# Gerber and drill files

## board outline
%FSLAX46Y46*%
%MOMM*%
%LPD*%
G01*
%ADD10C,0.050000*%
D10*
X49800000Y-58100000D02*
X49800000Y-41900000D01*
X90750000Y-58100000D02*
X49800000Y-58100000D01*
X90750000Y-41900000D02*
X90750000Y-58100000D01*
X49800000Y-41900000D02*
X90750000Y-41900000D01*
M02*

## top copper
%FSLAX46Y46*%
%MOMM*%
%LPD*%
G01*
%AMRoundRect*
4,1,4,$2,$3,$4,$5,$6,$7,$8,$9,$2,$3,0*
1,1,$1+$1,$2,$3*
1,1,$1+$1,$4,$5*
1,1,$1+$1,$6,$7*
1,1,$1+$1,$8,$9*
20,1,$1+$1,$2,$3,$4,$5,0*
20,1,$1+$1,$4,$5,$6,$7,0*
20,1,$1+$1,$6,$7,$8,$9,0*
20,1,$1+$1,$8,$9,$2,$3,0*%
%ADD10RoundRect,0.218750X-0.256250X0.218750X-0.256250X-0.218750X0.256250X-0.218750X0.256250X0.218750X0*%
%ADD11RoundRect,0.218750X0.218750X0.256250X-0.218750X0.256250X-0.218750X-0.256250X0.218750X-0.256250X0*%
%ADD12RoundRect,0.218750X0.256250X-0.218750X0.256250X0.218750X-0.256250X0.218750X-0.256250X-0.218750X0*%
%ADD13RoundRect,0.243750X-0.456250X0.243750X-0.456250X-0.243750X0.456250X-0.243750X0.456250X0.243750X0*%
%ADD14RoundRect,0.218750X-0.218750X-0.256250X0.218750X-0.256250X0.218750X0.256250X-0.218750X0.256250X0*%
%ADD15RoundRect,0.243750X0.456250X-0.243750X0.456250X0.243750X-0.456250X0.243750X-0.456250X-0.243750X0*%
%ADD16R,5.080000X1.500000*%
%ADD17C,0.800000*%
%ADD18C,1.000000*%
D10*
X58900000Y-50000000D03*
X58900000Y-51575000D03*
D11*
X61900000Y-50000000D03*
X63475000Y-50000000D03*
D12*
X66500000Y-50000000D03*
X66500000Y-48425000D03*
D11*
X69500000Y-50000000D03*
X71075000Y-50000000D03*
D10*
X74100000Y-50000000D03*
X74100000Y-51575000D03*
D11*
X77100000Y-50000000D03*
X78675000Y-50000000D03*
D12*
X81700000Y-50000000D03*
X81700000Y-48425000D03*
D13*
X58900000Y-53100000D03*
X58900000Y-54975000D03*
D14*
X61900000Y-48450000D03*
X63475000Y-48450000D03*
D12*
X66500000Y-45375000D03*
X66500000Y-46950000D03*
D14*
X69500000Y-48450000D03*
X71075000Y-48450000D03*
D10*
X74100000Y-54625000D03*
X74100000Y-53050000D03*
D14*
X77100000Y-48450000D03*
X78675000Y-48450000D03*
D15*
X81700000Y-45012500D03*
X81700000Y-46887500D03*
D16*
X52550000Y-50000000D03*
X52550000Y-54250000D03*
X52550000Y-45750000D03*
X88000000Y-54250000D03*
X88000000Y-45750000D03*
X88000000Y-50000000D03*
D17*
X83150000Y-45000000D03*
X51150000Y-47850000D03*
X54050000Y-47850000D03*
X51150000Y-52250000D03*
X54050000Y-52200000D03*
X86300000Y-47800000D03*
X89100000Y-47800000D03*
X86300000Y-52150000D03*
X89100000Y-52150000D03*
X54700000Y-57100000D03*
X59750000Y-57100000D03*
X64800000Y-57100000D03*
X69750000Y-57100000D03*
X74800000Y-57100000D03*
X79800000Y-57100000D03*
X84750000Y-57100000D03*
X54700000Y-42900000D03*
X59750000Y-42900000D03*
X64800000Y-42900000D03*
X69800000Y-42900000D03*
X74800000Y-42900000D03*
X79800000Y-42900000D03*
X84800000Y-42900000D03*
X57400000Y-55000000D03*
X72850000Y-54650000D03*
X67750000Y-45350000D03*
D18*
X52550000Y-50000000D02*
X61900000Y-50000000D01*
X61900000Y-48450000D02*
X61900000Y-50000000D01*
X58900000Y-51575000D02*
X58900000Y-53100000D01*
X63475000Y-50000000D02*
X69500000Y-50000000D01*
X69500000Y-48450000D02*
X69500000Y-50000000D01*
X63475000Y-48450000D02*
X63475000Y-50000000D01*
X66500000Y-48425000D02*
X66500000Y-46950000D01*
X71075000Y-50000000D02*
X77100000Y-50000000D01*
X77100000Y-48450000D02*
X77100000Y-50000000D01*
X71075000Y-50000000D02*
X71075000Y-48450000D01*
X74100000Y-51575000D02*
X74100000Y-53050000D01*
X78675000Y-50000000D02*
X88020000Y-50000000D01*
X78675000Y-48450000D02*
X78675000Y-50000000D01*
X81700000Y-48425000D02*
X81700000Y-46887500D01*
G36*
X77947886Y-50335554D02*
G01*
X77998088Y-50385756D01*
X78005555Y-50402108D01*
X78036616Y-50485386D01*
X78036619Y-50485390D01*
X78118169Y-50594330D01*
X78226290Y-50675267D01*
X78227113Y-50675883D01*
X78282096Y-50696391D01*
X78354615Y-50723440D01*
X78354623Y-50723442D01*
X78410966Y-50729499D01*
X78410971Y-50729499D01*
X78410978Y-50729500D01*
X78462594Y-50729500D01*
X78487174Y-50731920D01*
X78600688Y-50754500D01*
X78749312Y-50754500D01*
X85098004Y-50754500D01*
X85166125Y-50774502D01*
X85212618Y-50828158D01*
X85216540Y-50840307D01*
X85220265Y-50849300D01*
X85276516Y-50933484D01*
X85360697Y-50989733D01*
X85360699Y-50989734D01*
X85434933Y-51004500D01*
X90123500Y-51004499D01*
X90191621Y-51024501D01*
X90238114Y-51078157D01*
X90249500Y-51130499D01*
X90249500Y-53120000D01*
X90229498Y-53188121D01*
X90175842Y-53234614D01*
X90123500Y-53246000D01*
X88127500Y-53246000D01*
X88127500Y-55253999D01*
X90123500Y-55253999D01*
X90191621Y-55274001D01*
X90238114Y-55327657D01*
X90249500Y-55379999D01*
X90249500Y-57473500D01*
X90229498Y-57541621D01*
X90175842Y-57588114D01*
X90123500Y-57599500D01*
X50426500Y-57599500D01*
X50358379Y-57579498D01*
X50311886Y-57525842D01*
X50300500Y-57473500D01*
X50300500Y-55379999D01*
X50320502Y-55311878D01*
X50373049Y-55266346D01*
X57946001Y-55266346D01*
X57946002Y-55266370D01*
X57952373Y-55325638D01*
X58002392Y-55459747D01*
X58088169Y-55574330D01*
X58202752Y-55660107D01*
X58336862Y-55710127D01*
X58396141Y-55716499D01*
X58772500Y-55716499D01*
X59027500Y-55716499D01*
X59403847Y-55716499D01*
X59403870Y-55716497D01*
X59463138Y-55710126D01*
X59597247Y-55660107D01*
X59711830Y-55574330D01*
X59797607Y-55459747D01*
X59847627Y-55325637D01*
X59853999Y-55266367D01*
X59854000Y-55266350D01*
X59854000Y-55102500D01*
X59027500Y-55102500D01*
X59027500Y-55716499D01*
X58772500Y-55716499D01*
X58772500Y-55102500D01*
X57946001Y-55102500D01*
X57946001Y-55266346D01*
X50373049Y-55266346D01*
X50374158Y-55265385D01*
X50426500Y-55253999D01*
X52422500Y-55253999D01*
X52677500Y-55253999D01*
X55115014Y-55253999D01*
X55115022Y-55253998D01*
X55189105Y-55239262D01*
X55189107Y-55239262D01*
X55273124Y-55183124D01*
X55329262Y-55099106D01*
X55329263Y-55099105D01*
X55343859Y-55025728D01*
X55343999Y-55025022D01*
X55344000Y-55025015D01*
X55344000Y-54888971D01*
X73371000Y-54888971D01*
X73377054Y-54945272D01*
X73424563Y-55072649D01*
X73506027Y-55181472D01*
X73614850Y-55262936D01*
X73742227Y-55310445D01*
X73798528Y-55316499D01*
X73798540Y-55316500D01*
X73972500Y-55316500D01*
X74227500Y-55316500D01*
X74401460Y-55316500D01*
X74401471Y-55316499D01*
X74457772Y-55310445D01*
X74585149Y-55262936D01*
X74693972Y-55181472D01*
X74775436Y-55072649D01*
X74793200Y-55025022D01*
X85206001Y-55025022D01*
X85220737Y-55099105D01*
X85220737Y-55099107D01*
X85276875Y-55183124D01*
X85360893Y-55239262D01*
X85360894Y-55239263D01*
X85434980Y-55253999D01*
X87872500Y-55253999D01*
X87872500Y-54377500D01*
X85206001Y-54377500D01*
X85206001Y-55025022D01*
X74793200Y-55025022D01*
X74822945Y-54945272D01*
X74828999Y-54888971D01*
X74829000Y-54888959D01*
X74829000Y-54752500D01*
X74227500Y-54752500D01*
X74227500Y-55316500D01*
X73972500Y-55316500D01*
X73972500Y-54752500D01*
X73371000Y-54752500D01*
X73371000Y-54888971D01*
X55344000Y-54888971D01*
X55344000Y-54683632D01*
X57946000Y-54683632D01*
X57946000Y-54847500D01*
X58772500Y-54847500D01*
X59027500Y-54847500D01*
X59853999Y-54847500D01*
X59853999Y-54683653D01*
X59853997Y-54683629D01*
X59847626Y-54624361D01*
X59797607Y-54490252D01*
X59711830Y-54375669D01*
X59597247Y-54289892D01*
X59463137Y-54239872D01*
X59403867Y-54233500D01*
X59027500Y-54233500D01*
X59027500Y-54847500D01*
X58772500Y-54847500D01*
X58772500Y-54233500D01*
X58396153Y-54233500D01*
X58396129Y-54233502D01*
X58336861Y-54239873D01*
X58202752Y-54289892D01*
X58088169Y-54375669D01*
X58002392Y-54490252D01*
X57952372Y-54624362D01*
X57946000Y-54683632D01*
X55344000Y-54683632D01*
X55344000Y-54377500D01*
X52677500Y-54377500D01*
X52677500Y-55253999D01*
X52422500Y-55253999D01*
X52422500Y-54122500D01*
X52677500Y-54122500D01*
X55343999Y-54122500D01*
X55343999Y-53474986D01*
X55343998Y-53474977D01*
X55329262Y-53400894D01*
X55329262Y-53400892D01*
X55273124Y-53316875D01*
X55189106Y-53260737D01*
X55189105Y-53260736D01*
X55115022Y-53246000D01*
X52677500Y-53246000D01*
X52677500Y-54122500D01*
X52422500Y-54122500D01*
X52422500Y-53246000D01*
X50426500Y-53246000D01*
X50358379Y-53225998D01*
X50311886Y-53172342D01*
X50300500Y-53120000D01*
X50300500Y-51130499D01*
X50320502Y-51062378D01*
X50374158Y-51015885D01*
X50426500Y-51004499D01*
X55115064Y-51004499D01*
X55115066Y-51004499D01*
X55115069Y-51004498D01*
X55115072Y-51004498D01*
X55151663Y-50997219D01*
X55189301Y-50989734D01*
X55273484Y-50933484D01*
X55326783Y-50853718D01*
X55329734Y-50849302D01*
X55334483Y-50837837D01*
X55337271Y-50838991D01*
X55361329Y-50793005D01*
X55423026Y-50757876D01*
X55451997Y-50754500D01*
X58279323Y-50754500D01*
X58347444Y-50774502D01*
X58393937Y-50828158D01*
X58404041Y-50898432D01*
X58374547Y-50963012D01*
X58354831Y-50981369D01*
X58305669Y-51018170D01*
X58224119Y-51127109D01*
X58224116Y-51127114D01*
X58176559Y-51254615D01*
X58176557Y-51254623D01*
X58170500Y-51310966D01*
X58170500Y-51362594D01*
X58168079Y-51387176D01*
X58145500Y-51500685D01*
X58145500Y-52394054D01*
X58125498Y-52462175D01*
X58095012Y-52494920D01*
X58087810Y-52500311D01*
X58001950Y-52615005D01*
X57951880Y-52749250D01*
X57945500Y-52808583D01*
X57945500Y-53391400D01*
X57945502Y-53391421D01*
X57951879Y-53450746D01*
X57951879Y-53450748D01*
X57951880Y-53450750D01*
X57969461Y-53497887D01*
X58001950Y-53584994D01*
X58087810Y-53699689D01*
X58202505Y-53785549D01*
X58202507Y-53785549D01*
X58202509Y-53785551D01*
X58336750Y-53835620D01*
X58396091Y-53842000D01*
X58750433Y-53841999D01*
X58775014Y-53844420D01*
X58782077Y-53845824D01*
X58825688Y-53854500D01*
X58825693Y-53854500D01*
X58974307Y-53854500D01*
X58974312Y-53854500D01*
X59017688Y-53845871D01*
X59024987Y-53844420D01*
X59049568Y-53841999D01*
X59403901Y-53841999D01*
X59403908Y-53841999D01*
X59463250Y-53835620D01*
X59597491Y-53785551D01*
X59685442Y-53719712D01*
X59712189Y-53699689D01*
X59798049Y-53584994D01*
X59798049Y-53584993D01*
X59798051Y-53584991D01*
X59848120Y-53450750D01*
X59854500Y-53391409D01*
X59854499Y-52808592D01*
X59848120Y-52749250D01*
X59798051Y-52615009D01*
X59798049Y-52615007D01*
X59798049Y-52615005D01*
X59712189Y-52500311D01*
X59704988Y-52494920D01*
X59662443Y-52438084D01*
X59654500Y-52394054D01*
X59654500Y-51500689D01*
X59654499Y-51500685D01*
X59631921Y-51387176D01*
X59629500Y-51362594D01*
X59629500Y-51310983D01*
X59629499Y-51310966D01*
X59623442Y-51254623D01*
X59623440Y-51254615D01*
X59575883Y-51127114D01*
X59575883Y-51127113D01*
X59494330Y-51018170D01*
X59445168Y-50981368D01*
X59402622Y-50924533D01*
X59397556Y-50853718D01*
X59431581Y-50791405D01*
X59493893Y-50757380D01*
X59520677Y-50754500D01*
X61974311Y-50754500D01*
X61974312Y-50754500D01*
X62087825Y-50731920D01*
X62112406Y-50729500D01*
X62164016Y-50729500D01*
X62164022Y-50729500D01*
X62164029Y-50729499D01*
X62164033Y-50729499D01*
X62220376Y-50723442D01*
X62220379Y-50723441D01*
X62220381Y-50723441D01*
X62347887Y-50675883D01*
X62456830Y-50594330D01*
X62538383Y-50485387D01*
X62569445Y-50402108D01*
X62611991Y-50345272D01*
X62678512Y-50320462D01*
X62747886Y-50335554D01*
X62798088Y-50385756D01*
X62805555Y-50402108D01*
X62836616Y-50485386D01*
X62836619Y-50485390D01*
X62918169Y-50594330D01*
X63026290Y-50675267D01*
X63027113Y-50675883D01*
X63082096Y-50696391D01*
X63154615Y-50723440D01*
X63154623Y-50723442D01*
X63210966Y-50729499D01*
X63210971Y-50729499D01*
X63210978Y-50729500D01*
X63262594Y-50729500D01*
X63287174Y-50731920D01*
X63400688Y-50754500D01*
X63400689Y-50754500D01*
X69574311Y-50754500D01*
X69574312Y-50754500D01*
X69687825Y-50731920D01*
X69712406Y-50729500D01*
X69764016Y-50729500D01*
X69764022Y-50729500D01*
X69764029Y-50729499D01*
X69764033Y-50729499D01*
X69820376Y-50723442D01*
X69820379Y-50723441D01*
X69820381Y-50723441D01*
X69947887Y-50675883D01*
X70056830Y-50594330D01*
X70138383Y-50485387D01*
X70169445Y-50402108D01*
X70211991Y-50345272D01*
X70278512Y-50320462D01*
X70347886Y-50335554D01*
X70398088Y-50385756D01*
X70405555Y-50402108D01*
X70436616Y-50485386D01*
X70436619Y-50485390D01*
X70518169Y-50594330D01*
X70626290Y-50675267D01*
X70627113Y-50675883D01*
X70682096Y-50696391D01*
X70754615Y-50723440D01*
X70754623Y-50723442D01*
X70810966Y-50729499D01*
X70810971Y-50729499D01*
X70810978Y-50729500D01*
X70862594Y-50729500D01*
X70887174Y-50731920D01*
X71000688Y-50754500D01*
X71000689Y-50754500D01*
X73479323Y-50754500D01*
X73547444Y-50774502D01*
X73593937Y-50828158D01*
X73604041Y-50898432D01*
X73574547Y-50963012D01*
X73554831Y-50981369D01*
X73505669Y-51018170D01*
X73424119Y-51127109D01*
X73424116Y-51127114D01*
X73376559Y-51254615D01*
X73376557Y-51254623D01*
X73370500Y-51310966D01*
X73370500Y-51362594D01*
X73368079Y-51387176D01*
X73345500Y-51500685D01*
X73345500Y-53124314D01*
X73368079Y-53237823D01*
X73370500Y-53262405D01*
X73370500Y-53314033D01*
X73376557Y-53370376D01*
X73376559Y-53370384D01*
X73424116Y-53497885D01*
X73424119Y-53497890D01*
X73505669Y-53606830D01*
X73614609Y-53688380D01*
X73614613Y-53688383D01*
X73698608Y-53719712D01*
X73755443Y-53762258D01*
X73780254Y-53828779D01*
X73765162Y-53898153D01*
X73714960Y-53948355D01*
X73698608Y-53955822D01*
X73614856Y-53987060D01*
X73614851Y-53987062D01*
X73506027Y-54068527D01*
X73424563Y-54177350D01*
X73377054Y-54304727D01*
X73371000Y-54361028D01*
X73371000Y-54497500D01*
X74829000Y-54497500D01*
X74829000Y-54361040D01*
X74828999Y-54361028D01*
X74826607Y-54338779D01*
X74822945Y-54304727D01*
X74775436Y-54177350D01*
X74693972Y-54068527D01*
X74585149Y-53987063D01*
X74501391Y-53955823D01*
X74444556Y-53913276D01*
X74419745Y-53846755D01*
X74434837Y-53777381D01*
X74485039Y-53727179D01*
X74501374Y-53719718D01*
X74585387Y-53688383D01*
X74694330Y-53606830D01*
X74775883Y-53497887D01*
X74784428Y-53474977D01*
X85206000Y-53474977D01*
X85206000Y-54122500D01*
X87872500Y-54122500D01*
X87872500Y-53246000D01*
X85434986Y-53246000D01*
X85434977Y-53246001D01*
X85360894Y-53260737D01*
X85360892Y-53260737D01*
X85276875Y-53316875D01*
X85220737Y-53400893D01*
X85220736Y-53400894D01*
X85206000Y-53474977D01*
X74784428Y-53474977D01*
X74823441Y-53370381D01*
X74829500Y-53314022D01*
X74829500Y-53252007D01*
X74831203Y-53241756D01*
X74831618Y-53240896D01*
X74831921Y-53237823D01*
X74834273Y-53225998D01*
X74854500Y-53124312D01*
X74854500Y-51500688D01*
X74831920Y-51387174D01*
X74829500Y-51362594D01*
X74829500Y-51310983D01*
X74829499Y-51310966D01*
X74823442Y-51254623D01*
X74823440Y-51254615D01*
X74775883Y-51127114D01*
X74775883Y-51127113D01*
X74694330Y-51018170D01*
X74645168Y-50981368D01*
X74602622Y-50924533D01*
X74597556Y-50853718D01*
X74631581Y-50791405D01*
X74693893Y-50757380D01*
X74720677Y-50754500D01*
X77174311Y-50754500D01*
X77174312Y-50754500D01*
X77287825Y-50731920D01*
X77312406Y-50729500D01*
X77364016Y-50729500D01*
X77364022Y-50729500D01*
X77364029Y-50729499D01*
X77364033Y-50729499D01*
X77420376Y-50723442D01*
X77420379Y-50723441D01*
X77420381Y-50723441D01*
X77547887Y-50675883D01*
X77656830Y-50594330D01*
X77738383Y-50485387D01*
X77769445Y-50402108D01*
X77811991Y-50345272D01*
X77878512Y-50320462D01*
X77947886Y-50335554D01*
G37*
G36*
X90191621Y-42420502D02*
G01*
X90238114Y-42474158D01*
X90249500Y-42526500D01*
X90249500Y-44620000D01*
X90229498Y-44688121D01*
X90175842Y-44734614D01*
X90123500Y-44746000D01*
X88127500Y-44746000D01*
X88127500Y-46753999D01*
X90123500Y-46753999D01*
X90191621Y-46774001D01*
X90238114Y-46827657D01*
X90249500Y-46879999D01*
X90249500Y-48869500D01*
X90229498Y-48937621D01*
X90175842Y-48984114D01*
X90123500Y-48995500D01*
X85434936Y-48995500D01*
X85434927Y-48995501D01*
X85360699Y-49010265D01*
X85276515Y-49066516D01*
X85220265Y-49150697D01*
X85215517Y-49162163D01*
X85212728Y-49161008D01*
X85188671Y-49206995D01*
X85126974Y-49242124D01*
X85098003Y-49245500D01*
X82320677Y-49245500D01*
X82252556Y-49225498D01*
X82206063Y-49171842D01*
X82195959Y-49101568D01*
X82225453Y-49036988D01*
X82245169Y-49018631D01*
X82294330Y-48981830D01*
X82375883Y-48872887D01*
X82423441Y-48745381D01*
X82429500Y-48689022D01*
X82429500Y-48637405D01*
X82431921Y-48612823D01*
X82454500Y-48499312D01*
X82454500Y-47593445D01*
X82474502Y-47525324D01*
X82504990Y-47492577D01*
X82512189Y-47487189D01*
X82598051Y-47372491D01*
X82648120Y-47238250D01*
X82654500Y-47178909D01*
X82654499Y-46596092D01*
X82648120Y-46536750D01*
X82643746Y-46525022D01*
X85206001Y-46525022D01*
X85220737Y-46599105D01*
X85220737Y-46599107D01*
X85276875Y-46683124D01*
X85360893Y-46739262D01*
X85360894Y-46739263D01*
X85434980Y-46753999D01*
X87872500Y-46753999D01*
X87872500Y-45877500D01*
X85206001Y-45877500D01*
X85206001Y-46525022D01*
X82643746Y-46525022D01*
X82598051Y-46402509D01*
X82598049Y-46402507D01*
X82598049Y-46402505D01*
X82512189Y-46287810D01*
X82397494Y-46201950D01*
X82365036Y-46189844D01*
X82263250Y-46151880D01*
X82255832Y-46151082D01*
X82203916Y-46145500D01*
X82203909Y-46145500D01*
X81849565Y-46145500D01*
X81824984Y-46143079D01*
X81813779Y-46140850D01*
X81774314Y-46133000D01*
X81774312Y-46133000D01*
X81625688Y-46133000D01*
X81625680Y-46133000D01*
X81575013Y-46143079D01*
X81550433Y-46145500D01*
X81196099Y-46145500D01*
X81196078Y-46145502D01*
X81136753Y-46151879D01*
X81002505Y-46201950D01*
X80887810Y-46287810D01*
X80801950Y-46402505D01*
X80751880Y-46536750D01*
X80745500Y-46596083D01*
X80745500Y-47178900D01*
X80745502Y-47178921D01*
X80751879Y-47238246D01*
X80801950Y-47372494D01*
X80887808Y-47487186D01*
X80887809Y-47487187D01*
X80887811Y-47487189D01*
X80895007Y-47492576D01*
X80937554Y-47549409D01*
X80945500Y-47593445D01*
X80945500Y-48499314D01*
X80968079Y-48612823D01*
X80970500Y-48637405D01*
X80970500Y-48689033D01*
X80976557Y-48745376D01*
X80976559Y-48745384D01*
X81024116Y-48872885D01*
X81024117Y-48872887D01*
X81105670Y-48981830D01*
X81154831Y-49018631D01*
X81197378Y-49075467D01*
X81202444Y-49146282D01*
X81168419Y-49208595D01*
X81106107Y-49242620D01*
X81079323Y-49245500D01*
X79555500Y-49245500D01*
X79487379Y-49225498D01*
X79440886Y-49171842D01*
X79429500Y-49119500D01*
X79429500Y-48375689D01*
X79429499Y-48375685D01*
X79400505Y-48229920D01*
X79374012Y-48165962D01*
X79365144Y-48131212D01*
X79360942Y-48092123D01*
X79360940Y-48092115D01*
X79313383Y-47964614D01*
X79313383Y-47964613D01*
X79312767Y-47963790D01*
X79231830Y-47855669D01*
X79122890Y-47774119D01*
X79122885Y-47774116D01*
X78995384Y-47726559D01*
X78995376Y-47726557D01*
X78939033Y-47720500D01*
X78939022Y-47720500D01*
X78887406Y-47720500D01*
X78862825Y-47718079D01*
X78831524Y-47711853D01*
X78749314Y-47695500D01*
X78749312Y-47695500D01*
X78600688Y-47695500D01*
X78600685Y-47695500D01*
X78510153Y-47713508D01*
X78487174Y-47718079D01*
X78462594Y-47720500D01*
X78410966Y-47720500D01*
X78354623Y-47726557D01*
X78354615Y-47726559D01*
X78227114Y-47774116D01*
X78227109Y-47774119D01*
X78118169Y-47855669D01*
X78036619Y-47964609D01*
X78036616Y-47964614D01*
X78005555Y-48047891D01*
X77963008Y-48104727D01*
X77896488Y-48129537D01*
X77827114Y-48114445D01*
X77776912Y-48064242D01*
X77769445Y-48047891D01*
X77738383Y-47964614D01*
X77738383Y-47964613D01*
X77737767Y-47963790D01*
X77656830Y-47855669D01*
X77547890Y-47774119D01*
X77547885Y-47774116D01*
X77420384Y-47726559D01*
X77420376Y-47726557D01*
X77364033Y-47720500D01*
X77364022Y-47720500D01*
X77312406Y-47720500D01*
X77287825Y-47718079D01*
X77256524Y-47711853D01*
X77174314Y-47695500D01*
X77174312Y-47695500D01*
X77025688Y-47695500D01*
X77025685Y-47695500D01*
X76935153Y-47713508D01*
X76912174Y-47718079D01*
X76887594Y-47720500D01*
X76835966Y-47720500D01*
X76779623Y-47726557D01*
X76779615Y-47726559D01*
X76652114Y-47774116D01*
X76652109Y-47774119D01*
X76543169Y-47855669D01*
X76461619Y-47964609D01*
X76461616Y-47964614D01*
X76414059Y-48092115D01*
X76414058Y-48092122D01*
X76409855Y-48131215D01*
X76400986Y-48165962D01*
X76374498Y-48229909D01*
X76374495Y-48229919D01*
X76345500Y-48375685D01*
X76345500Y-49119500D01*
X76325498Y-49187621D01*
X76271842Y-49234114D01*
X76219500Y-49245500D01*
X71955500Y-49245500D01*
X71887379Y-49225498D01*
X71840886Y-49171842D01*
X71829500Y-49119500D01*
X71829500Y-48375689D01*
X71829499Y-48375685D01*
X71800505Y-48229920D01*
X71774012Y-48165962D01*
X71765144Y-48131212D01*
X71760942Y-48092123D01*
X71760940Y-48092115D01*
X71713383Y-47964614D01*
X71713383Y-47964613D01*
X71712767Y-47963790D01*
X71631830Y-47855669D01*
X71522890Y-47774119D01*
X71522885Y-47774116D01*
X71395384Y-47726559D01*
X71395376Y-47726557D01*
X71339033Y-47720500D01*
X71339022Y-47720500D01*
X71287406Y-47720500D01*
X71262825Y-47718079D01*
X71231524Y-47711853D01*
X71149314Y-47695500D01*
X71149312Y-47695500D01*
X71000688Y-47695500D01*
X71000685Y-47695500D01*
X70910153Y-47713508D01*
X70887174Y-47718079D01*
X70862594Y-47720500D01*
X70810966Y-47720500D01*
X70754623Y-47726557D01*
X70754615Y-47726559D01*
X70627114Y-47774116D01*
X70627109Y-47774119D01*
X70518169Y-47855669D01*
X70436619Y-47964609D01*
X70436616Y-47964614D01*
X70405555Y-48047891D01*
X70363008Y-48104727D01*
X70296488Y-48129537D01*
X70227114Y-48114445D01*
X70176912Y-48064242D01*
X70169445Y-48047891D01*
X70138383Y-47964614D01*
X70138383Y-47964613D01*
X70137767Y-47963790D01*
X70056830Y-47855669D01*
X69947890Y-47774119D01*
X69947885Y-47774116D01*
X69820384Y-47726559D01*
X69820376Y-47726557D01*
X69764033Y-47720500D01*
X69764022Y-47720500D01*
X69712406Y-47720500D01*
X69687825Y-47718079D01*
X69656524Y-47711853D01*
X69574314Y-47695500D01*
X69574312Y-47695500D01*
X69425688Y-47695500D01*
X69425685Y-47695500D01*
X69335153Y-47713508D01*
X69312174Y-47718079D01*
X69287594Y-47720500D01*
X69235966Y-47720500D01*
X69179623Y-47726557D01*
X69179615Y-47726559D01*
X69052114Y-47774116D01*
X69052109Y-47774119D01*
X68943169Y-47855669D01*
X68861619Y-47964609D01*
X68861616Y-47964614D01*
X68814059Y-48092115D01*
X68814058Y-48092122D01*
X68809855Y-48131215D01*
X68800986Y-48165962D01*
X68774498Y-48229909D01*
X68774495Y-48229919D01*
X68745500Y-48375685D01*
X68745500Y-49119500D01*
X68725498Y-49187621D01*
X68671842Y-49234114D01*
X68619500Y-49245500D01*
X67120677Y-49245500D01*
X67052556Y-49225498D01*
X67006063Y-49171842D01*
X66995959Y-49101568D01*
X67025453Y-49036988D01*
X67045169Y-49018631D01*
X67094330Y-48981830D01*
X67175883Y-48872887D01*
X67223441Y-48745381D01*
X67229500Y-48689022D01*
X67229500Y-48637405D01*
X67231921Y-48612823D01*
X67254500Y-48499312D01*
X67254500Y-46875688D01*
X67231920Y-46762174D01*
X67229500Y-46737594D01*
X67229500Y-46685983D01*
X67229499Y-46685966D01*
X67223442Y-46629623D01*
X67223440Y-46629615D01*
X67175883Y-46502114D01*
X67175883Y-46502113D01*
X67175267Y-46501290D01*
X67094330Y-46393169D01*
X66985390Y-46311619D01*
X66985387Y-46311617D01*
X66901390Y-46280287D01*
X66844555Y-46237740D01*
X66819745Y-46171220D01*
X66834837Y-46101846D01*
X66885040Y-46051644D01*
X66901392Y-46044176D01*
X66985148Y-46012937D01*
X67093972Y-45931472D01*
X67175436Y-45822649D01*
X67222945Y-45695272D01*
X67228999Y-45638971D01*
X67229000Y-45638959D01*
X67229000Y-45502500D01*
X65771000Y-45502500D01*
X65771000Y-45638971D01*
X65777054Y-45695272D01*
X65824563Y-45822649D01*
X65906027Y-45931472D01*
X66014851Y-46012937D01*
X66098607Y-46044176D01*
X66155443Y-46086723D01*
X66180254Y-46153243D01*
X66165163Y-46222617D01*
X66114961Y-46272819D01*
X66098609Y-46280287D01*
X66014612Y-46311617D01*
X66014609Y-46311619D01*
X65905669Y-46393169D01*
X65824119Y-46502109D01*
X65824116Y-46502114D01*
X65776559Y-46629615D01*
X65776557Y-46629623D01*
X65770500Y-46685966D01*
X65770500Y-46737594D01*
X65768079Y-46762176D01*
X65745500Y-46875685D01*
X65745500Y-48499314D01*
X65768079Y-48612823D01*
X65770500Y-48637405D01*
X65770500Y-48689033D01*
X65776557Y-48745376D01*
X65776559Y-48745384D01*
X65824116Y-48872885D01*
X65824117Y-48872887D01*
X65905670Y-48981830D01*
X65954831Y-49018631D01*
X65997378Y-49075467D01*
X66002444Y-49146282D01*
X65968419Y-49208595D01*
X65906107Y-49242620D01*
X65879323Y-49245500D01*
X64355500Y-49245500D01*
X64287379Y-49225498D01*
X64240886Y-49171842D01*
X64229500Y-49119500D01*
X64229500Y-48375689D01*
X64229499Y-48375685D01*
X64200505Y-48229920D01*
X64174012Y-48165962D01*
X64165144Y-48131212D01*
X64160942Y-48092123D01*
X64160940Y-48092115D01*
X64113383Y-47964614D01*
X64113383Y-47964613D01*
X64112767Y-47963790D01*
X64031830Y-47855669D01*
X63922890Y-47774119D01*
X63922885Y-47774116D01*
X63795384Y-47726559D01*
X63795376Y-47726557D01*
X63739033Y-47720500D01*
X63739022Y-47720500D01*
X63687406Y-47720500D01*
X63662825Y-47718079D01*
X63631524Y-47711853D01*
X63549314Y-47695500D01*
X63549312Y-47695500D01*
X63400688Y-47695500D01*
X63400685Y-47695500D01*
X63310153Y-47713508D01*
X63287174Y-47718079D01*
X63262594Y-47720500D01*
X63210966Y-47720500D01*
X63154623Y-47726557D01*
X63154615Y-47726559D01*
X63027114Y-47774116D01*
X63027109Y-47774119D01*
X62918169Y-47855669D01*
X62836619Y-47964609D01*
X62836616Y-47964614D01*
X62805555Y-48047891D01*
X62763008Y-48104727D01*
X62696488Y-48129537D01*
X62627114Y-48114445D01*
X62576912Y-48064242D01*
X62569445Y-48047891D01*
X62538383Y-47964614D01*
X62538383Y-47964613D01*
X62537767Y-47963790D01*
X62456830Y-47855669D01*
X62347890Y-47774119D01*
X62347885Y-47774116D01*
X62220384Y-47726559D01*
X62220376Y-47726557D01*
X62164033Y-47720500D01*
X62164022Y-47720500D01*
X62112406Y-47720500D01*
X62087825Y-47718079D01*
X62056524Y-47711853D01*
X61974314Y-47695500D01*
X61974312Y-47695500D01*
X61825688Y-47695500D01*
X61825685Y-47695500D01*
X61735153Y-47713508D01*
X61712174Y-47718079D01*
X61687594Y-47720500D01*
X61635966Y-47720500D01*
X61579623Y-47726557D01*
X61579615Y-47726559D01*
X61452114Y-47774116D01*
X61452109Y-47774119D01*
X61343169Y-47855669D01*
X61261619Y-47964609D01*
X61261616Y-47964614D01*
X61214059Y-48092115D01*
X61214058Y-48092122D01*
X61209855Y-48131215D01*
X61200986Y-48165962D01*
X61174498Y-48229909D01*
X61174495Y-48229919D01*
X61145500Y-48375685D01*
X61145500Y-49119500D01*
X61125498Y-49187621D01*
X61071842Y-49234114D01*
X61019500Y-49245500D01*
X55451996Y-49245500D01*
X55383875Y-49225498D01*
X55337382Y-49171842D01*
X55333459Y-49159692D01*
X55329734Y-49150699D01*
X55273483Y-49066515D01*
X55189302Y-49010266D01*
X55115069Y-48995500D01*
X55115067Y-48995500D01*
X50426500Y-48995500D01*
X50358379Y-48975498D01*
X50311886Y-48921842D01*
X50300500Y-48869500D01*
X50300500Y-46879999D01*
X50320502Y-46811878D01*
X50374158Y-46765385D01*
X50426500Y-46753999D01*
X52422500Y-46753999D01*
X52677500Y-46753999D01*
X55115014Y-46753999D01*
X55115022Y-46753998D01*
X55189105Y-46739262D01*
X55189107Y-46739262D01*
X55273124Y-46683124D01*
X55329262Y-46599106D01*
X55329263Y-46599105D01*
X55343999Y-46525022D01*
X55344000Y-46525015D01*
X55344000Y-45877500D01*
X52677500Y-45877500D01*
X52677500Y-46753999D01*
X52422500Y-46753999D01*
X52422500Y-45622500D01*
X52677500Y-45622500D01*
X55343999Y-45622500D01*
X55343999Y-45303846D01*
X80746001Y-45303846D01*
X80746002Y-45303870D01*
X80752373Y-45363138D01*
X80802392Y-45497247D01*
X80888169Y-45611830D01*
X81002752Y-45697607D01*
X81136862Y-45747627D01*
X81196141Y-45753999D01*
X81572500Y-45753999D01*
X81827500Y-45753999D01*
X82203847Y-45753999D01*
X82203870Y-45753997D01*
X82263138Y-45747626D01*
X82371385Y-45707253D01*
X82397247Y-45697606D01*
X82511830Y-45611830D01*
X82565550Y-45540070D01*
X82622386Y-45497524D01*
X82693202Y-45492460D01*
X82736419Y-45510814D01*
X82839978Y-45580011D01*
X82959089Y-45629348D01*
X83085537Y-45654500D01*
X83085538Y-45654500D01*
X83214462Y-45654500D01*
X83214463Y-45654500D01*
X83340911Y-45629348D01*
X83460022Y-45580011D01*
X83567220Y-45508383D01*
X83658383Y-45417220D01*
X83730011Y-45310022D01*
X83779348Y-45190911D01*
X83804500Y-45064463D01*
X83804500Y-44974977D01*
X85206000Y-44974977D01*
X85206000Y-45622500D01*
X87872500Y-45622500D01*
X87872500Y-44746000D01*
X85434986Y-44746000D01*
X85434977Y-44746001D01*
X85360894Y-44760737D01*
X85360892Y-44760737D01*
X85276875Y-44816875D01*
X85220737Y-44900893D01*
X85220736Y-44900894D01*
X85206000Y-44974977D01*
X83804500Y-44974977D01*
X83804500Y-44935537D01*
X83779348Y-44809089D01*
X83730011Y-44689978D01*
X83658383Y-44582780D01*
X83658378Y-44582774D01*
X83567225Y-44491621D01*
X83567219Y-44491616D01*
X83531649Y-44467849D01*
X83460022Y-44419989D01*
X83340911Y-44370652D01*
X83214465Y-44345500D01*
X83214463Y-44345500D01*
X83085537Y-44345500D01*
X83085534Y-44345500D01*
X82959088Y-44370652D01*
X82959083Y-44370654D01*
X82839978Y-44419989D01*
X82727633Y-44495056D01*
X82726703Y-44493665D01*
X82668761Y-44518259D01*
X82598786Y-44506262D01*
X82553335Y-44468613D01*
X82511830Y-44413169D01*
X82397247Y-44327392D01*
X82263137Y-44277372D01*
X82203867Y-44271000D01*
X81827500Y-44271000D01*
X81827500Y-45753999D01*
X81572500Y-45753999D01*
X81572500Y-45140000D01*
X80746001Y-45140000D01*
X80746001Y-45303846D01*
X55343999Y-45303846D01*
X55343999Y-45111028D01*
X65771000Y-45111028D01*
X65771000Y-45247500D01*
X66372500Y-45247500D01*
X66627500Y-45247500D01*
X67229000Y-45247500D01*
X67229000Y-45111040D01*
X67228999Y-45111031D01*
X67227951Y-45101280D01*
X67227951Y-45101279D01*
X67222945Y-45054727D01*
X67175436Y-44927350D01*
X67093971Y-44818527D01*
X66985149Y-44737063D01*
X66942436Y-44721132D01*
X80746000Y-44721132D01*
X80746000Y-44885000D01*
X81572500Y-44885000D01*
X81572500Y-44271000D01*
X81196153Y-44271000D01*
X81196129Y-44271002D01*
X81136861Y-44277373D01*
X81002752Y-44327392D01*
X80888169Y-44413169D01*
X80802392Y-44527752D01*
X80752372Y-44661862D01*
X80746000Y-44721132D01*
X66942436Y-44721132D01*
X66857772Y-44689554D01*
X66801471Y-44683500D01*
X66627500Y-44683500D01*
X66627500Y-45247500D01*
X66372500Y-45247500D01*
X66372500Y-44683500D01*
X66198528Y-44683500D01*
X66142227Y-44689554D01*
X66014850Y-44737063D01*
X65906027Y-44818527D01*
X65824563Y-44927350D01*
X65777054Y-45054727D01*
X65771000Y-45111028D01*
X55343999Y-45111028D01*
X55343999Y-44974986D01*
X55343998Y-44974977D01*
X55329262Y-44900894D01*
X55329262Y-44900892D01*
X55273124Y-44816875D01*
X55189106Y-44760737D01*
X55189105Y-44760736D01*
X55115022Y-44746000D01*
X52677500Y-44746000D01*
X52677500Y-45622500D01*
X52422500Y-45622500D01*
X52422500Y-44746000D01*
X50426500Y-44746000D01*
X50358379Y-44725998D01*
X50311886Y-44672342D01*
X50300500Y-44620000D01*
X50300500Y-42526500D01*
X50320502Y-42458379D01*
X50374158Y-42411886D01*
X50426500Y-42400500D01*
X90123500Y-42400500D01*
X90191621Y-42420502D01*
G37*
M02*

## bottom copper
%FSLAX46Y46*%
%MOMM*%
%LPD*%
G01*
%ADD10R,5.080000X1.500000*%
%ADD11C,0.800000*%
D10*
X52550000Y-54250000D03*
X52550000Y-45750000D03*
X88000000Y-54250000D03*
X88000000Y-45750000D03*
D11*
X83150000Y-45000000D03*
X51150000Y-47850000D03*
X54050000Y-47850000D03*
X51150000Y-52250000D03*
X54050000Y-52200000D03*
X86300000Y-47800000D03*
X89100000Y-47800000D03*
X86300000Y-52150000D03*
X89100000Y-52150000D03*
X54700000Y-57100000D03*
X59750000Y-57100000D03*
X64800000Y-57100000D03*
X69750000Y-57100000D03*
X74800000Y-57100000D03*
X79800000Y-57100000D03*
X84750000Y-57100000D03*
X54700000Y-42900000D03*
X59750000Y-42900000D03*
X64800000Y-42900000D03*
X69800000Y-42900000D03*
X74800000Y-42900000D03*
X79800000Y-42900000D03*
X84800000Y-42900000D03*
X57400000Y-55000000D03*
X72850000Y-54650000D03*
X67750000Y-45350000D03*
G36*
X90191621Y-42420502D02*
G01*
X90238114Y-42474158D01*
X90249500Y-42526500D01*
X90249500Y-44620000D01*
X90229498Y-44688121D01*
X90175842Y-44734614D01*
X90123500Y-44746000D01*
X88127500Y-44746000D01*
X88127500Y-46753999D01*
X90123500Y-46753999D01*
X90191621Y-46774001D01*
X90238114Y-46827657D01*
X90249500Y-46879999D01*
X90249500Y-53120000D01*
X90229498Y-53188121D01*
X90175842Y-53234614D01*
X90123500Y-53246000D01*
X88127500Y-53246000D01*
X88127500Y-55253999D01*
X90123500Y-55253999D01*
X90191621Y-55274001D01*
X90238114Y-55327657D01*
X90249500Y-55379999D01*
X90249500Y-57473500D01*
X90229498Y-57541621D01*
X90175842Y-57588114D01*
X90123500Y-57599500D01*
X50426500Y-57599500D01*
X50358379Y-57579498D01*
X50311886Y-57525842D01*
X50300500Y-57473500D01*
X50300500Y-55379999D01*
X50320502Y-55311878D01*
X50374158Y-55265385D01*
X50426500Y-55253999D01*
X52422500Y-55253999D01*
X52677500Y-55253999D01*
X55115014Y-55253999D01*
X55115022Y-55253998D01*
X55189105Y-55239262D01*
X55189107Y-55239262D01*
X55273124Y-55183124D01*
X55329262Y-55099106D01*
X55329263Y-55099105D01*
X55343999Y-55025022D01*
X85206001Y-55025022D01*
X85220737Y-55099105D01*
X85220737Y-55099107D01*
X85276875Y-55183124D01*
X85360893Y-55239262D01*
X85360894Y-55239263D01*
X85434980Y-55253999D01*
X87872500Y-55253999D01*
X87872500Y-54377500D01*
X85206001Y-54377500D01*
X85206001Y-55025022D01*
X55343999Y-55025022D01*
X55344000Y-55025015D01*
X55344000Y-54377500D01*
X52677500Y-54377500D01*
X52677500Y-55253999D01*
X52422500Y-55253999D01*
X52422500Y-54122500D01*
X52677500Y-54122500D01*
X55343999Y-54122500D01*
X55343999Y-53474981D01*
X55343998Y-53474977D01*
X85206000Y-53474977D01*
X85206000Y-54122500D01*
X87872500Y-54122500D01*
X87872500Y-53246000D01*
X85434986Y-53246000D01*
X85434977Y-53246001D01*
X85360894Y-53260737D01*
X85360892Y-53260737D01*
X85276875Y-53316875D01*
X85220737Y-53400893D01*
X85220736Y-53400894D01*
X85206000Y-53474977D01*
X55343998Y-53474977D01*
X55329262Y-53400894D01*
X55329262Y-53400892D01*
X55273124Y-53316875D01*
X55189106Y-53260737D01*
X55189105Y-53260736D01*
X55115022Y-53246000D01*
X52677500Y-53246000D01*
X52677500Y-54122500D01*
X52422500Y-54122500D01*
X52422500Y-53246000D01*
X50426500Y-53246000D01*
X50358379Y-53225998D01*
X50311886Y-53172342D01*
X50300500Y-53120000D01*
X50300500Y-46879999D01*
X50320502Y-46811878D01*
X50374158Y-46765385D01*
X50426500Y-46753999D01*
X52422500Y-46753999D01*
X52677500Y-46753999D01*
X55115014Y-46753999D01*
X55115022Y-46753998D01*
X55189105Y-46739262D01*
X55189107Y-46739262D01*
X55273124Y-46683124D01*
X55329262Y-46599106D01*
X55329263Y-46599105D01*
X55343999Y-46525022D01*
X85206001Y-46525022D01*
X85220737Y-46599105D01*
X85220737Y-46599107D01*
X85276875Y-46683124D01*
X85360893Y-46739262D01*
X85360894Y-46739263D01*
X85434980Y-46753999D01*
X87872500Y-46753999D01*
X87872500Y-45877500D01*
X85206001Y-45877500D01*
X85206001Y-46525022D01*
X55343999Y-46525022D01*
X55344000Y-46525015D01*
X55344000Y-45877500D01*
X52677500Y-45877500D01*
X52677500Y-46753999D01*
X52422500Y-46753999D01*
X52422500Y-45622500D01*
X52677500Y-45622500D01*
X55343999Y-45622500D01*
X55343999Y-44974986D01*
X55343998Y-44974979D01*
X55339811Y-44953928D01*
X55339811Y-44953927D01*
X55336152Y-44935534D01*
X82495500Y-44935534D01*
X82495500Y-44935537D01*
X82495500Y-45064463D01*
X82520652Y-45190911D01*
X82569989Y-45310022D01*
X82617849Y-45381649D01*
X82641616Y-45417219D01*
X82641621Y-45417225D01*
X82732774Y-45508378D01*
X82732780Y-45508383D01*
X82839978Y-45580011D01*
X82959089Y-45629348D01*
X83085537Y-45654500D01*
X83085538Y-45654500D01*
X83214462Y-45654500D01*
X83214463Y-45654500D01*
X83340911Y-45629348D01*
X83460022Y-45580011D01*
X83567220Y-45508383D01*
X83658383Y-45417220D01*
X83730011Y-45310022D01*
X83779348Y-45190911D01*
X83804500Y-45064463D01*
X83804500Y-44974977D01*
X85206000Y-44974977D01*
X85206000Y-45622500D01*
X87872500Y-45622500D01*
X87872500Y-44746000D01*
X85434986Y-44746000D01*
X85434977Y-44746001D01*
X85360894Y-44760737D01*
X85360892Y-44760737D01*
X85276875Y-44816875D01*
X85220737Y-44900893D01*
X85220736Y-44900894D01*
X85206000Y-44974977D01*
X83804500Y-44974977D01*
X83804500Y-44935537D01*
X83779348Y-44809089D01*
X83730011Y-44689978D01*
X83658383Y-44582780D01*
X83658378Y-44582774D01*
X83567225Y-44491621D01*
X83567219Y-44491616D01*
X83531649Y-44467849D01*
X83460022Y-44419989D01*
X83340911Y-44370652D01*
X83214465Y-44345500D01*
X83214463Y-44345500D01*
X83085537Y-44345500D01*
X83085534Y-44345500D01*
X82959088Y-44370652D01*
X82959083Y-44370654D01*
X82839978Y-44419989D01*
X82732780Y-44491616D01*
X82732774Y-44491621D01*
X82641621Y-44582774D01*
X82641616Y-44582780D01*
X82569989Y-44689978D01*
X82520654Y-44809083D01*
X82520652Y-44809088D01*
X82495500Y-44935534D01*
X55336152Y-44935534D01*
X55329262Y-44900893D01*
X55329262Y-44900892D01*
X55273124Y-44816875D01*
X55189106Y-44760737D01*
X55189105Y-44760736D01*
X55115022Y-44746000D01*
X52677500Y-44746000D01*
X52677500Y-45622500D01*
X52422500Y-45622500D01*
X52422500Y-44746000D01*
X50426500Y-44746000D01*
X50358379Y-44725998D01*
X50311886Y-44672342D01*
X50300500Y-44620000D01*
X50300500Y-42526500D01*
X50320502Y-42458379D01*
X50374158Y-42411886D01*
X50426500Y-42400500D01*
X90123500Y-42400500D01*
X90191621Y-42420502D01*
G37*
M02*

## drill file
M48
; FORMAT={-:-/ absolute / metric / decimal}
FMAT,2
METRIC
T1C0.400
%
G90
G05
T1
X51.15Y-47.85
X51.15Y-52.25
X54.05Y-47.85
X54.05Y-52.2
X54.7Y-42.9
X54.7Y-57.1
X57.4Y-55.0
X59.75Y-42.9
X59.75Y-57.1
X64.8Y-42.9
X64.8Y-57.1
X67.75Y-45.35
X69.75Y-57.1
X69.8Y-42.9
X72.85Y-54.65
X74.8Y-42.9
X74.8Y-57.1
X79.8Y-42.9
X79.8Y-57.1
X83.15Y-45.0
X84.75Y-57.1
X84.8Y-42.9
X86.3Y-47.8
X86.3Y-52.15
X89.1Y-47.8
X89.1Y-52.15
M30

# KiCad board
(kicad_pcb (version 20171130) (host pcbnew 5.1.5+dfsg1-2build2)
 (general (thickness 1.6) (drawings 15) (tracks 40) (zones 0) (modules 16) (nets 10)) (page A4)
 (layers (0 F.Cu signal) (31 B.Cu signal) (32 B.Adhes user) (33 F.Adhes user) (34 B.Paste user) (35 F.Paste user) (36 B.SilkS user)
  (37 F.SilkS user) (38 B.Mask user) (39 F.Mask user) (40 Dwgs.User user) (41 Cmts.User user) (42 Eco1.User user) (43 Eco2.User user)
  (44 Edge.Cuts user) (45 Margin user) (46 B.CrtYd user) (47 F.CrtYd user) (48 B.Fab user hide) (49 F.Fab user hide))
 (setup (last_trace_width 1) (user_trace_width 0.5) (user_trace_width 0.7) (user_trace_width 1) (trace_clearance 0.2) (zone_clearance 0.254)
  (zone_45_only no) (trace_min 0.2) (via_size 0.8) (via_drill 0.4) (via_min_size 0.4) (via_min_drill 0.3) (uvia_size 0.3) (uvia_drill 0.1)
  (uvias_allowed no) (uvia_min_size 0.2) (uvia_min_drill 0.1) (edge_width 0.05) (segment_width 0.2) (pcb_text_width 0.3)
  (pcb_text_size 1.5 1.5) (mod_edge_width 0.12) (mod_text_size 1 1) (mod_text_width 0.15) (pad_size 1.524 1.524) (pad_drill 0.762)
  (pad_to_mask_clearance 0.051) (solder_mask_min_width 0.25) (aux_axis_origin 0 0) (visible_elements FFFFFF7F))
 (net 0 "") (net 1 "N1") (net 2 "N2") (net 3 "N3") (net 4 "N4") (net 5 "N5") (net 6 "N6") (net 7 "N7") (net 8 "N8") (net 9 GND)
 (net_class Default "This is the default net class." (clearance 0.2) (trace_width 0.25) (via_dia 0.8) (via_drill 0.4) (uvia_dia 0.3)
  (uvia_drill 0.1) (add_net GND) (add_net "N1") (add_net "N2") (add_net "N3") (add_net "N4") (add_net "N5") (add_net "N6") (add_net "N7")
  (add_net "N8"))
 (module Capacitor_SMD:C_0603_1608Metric (layer F.Cu) (at 58.9 50.7875 270)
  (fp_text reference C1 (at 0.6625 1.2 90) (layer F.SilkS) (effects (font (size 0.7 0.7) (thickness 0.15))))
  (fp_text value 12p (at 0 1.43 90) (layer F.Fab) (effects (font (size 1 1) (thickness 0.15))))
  (pad 1 smd roundrect (at -0.7875 0 270) (size 0.875 0.95) (layers F.Cu F.Paste F.Mask) (roundrect_rratio 0.25) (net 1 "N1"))
  (pad 2 smd roundrect (at 0.7875 0 270) (size 0.875 0.95) (layers F.Cu F.Paste F.Mask) (roundrect_rratio 0.25) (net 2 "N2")))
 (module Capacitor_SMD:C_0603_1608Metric (layer F.Cu) (at 62.6875 50 180)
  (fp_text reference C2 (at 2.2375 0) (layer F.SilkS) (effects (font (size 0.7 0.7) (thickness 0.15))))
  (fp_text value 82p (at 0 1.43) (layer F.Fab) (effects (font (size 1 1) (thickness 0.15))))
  (pad 2 smd roundrect (at 0.7875 0 180) (size 0.875 0.95) (layers F.Cu F.Paste F.Mask) (roundrect_rratio 0.25) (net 1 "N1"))
  (pad 1 smd roundrect (at -0.7875 0 180) (size 0.875 0.95) (layers F.Cu F.Paste F.Mask) (roundrect_rratio 0.25) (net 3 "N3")))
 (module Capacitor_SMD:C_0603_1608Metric (layer F.Cu) (at 66.5 49.2125 90)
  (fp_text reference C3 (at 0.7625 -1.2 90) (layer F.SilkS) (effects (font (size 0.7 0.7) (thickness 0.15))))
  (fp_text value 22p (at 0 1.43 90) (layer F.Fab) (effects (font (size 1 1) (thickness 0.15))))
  (pad 1 smd roundrect (at -0.7875 0 90) (size 0.875 0.95) (layers F.Cu F.Paste F.Mask) (roundrect_rratio 0.25) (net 3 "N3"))
  (pad 2 smd roundrect (at 0.7875 0 90) (size 0.875 0.95) (layers F.Cu F.Paste F.Mask) (roundrect_rratio 0.25) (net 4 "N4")))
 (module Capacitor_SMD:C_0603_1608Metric (layer F.Cu) (at 70.2875 50 180)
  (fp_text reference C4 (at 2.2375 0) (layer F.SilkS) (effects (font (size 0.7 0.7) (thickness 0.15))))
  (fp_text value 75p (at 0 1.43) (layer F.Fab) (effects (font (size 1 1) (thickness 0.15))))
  (pad 2 smd roundrect (at 0.7875 0 180) (size 0.875 0.95) (layers F.Cu F.Paste F.Mask) (roundrect_rratio 0.25) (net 3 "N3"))
  (pad 1 smd roundrect (at -0.7875 0 180) (size 0.875 0.95) (layers F.Cu F.Paste F.Mask) (roundrect_rratio 0.25) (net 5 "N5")))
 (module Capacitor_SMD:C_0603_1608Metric (layer F.Cu) (at 74.1 50.7875 270)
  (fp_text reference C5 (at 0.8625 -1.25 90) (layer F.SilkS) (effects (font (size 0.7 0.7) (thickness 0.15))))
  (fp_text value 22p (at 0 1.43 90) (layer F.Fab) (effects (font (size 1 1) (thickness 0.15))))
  (pad 1 smd roundrect (at -0.7875 0 270) (size 0.875 0.95) (layers F.Cu F.Paste F.Mask) (roundrect_rratio 0.25) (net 5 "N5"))
  (pad 2 smd roundrect (at 0.7875 0 270) (size 0.875 0.95) (layers F.Cu F.Paste F.Mask) (roundrect_rratio 0.25) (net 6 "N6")))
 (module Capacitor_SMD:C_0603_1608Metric (layer F.Cu) (at 77.8875 50 180)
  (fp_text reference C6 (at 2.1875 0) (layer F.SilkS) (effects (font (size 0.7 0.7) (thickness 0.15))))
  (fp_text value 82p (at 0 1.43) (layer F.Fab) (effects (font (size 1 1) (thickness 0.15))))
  (pad 2 smd roundrect (at 0.7875 0 180) (size 0.875 0.95) (layers F.Cu F.Paste F.Mask) (roundrect_rratio 0.25) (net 5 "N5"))
  (pad 1 smd roundrect (at -0.7875 0 180) (size 0.875 0.95) (layers F.Cu F.Paste F.Mask) (roundrect_rratio 0.25) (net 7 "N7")))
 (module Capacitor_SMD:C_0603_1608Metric (layer F.Cu) (at 81.7 49.2125 90)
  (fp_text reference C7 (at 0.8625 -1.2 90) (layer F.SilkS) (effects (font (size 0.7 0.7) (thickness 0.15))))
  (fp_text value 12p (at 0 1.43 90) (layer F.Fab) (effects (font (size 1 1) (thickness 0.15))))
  (pad 1 smd roundrect (at -0.7875 0 90) (size 0.875 0.95) (layers F.Cu F.Paste F.Mask) (roundrect_rratio 0.25) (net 7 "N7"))
  (pad 2 smd roundrect (at 0.7875 0 90) (size 0.875 0.95) (layers F.Cu F.Paste F.Mask) (roundrect_rratio 0.25) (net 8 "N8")))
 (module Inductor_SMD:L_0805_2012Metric (layer F.Cu) (at 58.9 54.0375 270)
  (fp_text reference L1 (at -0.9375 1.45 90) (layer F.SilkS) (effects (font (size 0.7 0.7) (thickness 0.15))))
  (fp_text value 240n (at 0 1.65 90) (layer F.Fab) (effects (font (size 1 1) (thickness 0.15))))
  (pad 1 smd roundrect (at -0.9375 0 270) (size 0.975 1.4) (layers F.Cu F.Paste F.Mask) (roundrect_rratio 0.25) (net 2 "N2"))
  (pad 2 smd roundrect (at 0.9375 0 270) (size 0.975 1.4) (layers F.Cu F.Paste F.Mask) (roundrect_rratio 0.25) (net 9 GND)))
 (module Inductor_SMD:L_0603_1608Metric (layer F.Cu) (at 62.6875 48.45)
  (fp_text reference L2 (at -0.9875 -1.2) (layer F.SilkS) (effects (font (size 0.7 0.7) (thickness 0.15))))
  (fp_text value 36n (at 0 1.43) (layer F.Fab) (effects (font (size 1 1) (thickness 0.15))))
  (pad 1 smd roundrect (at -0.7875 0) (size 0.875 0.95) (layers F.Cu F.Paste F.Mask) (roundrect_rratio 0.25) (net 1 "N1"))
  (pad 2 smd roundrect (at 0.7875 0) (size 0.875 0.95) (layers F.Cu F.Paste F.Mask) (roundrect_rratio 0.25) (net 3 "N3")))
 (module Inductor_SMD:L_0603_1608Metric (layer F.Cu) (at 66.5 46.1625 90)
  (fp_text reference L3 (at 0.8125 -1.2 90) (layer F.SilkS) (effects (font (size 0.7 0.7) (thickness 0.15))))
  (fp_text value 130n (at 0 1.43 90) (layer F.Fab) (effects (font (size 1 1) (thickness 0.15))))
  (pad 2 smd roundrect (at 0.7875 0 90) (size 0.875 0.95) (layers F.Cu F.Paste F.Mask) (roundrect_rratio 0.25) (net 9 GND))
  (pad 1 smd roundrect (at -0.7875 0 90) (size 0.875 0.95) (layers F.Cu F.Paste F.Mask) (roundrect_rratio 0.25) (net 4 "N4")))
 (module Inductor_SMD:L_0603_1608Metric (layer F.Cu) (at 70.2875 48.45)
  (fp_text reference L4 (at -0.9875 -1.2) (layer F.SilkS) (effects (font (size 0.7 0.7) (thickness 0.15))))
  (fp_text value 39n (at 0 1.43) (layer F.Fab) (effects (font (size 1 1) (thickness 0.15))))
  (pad 1 smd roundrect (at -0.7875 0) (size 0.875 0.95) (layers F.Cu F.Paste F.Mask) (roundrect_rratio 0.25) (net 3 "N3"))
  (pad 2 smd roundrect (at 0.7875 0) (size 0.875 0.95) (layers F.Cu F.Paste F.Mask) (roundrect_rratio 0.25) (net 5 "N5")))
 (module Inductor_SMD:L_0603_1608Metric (layer F.Cu) (at 74.1 53.8375 270)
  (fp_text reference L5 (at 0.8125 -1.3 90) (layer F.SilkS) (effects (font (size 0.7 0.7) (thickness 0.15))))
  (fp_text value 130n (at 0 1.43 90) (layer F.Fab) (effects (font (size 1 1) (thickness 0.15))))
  (pad 2 smd roundrect (at 0.7875 0 270) (size 0.875 0.95) (layers F.Cu F.Paste F.Mask) (roundrect_rratio 0.25) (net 9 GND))
  (pad 1 smd roundrect (at -0.7875 0 270) (size 0.875 0.95) (layers F.Cu F.Paste F.Mask) (roundrect_rratio 0.25) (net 6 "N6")))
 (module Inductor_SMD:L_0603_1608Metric (layer F.Cu) (at 77.8875 48.45)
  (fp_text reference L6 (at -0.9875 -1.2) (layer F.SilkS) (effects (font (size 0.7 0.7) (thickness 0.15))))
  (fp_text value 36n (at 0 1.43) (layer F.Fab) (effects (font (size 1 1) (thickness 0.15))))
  (pad 1 smd roundrect (at -0.7875 0) (size 0.875 0.95) (layers F.Cu F.Paste F.Mask) (roundrect_rratio 0.25) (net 5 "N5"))
  (pad 2 smd roundrect (at 0.7875 0) (size 0.875 0.95) (layers F.Cu F.Paste F.Mask) (roundrect_rratio 0.25) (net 7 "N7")))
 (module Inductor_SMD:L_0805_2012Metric (layer F.Cu) (at 81.7 45.95 90)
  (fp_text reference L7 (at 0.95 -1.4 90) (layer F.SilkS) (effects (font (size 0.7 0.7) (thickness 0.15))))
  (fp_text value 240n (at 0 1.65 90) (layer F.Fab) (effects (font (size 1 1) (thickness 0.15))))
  (pad 2 smd roundrect (at 0.9375 0 90) (size 0.975 1.4) (layers F.Cu F.Paste F.Mask) (roundrect_rratio 0.25) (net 9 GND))
  (pad 1 smd roundrect (at -0.9375 0 90) (size 0.975 1.4) (layers F.Cu F.Paste F.Mask) (roundrect_rratio 0.25) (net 8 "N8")))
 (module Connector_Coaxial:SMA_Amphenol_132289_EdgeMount (layer F.Cu) (at 52.55 50 180)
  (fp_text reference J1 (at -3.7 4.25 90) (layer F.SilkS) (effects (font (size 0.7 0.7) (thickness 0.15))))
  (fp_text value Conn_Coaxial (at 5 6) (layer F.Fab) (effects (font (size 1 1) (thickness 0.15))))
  (pad 1 smd rect (at 0 0 270) (size 1.5 5.08) (layers F.Cu F.Paste F.Mask) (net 1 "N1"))
  (pad 2 smd rect (at 0 -4.25 270) (size 1.5 5.08) (layers F.Cu F.Paste F.Mask) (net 9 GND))
  (pad 2 smd rect (at 0 4.25 270) (size 1.5 5.08) (layers F.Cu F.Paste F.Mask) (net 9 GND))
  (pad 2 smd rect (at 0 -4.25 270) (size 1.5 5.08) (layers B.Cu B.Paste B.Mask) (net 9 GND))
  (pad 2 smd rect (at 0 4.25 270) (size 1.5 5.08) (layers B.Cu B.Paste B.Mask) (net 9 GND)))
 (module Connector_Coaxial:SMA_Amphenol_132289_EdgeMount (layer F.Cu) (at 88 50)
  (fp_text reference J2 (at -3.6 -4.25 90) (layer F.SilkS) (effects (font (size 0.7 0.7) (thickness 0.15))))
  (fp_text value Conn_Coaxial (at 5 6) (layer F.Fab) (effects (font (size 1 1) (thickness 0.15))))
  (pad 2 smd rect (at 0 4.25 90) (size 1.5 5.08) (layers B.Cu B.Paste B.Mask) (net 9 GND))
  (pad 2 smd rect (at 0 -4.25 90) (size 1.5 5.08) (layers B.Cu B.Paste B.Mask) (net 9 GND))
  (pad 2 smd rect (at 0 4.25 90) (size 1.5 5.08) (layers F.Cu F.Paste F.Mask) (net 9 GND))
  (pad 2 smd rect (at 0 -4.25 90) (size 1.5 5.08) (layers F.Cu F.Paste F.Mask) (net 9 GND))
  (pad 1 smd rect (at 0 0 90) (size 1.5 5.08) (layers F.Cu F.Paste F.Mask) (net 7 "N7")))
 (gr_line (start 49.8 58.1) (end 49.8 41.9) (layer Edge.Cuts) (width 0.05))
 (gr_line (start 90.75 58.1) (end 49.8 58.1) (layer Edge.Cuts) (width 0.05))
 (gr_line (start 90.75 41.9) (end 90.75 58.1) (layer Edge.Cuts) (width 0.05))
 (gr_line (start 49.8 41.9) (end 90.75 41.9) (layer Edge.Cuts) (width 0.05))
 (via (at 83.15 45) (size 0.8) (drill 0.4) (layers F.Cu B.Cu) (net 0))
 (segment (start 52.55 50) (end 61.9 50) (width 1) (layer F.Cu) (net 1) (status 20))
 (segment (start 61.9 48.45) (end 61.9 50) (width 1) (layer F.Cu) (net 1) (status 30))
 (segment (start 58.9 51.575) (end 58.9 53.1) (width 1) (layer F.Cu) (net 2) (status 30))
 (segment (start 63.475 50) (end 69.5 50) (width 1) (layer F.Cu) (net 3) (status 30))
 (segment (start 69.5 48.45) (end 69.5 50) (width 1) (layer F.Cu) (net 3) (status 30))
 (segment (start 63.475 48.45) (end 63.475 50) (width 1) (layer F.Cu) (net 3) (status 30))
 (segment (start 66.5 48.425) (end 66.5 46.95) (width 1) (layer F.Cu) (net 4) (status 30))
 (segment (start 71.075 50) (end 77.1 50) (width 1) (layer F.Cu) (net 5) (status 30))
 (segment (start 77.1 48.45) (end 77.1 50) (width 1) (layer F.Cu) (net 5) (status 30))
 (segment (start 71.075 50) (end 71.075 48.45) (width 1) (layer F.Cu) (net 5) (status 30))
 (segment (start 74.1 51.575) (end 74.1 53.05) (width 1) (layer F.Cu) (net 6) (status 30))
 (segment (start 78.675 50) (end 88.02 50) (width 1) (layer F.Cu) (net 7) (status 10))
 (segment (start 78.675 48.45) (end 78.675 50) (width 1) (layer F.Cu) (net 7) (status 30))
 (segment (start 81.7 48.425) (end 81.7 46.8875) (width 1) (layer F.Cu) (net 8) (status 30))
 (via (at 51.15 47.85) (size 0.8) (drill 0.4) (layers F.Cu B.Cu) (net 9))
 (via (at 54.05 47.85) (size 0.8) (drill 0.4) (layers F.Cu B.Cu) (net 9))
 (via (at 51.15 52.25) (size 0.8) (drill 0.4) (layers F.Cu B.Cu) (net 9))
 (via (at 54.05 52.2) (size 0.8) (drill 0.4) (layers F.Cu B.Cu) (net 9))
 (via (at 86.3 47.8) (size 0.8) (drill 0.4) (layers F.Cu B.Cu) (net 9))
 (via (at 89.1 47.8) (size 0.8) (drill 0.4) (layers F.Cu B.Cu) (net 9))
 (via (at 86.3 52.15) (size 0.8) (drill 0.4) (layers F.Cu B.Cu) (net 9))
 (via (at 89.1 52.15) (size 0.8) (drill 0.4) (layers F.Cu B.Cu) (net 9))
 (via (at 54.7 57.1) (size 0.8) (drill 0.4) (layers F.Cu B.Cu) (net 9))
 (via (at 59.75 57.1) (size 0.8) (drill 0.4) (layers F.Cu B.Cu) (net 9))
 (via (at 64.8 57.1) (size 0.8) (drill 0.4) (layers F.Cu B.Cu) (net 9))
 (via (at 69.75 57.1) (size 0.8) (drill 0.4) (layers F.Cu B.Cu) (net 9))
 (via (at 74.8 57.1) (size 0.8) (drill 0.4) (layers F.Cu B.Cu) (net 9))
 (via (at 79.8 57.1) (size 0.8) (drill 0.4) (layers F.Cu B.Cu) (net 9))
 (via (at 84.75 57.1) (size 0.8) (drill 0.4) (layers F.Cu B.Cu) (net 9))
 (via (at 54.7 42.9) (size 0.8) (drill 0.4) (layers F.Cu B.Cu) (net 9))
 (via (at 59.75 42.9) (size 0.8) (drill 0.4) (layers F.Cu B.Cu) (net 9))
 (via (at 64.8 42.9) (size 0.8) (drill 0.4) (layers F.Cu B.Cu) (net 9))
 (via (at 69.8 42.9) (size 0.8) (drill 0.4) (layers F.Cu B.Cu) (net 9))
 (via (at 74.8 42.9) (size 0.8) (drill 0.4) (layers F.Cu B.Cu) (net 9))
 (via (at 79.8 42.9) (size 0.8) (drill 0.4) (layers F.Cu B.Cu) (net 9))
 (via (at 84.8 42.9) (size 0.8) (drill 0.4) (layers F.Cu B.Cu) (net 9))
 (via (at 57.4 55) (size 0.8) (drill 0.4) (layers F.Cu B.Cu) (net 9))
 (via (at 72.85 54.65) (size 0.8) (drill 0.4) (layers F.Cu B.Cu) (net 9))
 (via (at 67.75 45.35) (size 0.8) (drill 0.4) (layers F.Cu B.Cu) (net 9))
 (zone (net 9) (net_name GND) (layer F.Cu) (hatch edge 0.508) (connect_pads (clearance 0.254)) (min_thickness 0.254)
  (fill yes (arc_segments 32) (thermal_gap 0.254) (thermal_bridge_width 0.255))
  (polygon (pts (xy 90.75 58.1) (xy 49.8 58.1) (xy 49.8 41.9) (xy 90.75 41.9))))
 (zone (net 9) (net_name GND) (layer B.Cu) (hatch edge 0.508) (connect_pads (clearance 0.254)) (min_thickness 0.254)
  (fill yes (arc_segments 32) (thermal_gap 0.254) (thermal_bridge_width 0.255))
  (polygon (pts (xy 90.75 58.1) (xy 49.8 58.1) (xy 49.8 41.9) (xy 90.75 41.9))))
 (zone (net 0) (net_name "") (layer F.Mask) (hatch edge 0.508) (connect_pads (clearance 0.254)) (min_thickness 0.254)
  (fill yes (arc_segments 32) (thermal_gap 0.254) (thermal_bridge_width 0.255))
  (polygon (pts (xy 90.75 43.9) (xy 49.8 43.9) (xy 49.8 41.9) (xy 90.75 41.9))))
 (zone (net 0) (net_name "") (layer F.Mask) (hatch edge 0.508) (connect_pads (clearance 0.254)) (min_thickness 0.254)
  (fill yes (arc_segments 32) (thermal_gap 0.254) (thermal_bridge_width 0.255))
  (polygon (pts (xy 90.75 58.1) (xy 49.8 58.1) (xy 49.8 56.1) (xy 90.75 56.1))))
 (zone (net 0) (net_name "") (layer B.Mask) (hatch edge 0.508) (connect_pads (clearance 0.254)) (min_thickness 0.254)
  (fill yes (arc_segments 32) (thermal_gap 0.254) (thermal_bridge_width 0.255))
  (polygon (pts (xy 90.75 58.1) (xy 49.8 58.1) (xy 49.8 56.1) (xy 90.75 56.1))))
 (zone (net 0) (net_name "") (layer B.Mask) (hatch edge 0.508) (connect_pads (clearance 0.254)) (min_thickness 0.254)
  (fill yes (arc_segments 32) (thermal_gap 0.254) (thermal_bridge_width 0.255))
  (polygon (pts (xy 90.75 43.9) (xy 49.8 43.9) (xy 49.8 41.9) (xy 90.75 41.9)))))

